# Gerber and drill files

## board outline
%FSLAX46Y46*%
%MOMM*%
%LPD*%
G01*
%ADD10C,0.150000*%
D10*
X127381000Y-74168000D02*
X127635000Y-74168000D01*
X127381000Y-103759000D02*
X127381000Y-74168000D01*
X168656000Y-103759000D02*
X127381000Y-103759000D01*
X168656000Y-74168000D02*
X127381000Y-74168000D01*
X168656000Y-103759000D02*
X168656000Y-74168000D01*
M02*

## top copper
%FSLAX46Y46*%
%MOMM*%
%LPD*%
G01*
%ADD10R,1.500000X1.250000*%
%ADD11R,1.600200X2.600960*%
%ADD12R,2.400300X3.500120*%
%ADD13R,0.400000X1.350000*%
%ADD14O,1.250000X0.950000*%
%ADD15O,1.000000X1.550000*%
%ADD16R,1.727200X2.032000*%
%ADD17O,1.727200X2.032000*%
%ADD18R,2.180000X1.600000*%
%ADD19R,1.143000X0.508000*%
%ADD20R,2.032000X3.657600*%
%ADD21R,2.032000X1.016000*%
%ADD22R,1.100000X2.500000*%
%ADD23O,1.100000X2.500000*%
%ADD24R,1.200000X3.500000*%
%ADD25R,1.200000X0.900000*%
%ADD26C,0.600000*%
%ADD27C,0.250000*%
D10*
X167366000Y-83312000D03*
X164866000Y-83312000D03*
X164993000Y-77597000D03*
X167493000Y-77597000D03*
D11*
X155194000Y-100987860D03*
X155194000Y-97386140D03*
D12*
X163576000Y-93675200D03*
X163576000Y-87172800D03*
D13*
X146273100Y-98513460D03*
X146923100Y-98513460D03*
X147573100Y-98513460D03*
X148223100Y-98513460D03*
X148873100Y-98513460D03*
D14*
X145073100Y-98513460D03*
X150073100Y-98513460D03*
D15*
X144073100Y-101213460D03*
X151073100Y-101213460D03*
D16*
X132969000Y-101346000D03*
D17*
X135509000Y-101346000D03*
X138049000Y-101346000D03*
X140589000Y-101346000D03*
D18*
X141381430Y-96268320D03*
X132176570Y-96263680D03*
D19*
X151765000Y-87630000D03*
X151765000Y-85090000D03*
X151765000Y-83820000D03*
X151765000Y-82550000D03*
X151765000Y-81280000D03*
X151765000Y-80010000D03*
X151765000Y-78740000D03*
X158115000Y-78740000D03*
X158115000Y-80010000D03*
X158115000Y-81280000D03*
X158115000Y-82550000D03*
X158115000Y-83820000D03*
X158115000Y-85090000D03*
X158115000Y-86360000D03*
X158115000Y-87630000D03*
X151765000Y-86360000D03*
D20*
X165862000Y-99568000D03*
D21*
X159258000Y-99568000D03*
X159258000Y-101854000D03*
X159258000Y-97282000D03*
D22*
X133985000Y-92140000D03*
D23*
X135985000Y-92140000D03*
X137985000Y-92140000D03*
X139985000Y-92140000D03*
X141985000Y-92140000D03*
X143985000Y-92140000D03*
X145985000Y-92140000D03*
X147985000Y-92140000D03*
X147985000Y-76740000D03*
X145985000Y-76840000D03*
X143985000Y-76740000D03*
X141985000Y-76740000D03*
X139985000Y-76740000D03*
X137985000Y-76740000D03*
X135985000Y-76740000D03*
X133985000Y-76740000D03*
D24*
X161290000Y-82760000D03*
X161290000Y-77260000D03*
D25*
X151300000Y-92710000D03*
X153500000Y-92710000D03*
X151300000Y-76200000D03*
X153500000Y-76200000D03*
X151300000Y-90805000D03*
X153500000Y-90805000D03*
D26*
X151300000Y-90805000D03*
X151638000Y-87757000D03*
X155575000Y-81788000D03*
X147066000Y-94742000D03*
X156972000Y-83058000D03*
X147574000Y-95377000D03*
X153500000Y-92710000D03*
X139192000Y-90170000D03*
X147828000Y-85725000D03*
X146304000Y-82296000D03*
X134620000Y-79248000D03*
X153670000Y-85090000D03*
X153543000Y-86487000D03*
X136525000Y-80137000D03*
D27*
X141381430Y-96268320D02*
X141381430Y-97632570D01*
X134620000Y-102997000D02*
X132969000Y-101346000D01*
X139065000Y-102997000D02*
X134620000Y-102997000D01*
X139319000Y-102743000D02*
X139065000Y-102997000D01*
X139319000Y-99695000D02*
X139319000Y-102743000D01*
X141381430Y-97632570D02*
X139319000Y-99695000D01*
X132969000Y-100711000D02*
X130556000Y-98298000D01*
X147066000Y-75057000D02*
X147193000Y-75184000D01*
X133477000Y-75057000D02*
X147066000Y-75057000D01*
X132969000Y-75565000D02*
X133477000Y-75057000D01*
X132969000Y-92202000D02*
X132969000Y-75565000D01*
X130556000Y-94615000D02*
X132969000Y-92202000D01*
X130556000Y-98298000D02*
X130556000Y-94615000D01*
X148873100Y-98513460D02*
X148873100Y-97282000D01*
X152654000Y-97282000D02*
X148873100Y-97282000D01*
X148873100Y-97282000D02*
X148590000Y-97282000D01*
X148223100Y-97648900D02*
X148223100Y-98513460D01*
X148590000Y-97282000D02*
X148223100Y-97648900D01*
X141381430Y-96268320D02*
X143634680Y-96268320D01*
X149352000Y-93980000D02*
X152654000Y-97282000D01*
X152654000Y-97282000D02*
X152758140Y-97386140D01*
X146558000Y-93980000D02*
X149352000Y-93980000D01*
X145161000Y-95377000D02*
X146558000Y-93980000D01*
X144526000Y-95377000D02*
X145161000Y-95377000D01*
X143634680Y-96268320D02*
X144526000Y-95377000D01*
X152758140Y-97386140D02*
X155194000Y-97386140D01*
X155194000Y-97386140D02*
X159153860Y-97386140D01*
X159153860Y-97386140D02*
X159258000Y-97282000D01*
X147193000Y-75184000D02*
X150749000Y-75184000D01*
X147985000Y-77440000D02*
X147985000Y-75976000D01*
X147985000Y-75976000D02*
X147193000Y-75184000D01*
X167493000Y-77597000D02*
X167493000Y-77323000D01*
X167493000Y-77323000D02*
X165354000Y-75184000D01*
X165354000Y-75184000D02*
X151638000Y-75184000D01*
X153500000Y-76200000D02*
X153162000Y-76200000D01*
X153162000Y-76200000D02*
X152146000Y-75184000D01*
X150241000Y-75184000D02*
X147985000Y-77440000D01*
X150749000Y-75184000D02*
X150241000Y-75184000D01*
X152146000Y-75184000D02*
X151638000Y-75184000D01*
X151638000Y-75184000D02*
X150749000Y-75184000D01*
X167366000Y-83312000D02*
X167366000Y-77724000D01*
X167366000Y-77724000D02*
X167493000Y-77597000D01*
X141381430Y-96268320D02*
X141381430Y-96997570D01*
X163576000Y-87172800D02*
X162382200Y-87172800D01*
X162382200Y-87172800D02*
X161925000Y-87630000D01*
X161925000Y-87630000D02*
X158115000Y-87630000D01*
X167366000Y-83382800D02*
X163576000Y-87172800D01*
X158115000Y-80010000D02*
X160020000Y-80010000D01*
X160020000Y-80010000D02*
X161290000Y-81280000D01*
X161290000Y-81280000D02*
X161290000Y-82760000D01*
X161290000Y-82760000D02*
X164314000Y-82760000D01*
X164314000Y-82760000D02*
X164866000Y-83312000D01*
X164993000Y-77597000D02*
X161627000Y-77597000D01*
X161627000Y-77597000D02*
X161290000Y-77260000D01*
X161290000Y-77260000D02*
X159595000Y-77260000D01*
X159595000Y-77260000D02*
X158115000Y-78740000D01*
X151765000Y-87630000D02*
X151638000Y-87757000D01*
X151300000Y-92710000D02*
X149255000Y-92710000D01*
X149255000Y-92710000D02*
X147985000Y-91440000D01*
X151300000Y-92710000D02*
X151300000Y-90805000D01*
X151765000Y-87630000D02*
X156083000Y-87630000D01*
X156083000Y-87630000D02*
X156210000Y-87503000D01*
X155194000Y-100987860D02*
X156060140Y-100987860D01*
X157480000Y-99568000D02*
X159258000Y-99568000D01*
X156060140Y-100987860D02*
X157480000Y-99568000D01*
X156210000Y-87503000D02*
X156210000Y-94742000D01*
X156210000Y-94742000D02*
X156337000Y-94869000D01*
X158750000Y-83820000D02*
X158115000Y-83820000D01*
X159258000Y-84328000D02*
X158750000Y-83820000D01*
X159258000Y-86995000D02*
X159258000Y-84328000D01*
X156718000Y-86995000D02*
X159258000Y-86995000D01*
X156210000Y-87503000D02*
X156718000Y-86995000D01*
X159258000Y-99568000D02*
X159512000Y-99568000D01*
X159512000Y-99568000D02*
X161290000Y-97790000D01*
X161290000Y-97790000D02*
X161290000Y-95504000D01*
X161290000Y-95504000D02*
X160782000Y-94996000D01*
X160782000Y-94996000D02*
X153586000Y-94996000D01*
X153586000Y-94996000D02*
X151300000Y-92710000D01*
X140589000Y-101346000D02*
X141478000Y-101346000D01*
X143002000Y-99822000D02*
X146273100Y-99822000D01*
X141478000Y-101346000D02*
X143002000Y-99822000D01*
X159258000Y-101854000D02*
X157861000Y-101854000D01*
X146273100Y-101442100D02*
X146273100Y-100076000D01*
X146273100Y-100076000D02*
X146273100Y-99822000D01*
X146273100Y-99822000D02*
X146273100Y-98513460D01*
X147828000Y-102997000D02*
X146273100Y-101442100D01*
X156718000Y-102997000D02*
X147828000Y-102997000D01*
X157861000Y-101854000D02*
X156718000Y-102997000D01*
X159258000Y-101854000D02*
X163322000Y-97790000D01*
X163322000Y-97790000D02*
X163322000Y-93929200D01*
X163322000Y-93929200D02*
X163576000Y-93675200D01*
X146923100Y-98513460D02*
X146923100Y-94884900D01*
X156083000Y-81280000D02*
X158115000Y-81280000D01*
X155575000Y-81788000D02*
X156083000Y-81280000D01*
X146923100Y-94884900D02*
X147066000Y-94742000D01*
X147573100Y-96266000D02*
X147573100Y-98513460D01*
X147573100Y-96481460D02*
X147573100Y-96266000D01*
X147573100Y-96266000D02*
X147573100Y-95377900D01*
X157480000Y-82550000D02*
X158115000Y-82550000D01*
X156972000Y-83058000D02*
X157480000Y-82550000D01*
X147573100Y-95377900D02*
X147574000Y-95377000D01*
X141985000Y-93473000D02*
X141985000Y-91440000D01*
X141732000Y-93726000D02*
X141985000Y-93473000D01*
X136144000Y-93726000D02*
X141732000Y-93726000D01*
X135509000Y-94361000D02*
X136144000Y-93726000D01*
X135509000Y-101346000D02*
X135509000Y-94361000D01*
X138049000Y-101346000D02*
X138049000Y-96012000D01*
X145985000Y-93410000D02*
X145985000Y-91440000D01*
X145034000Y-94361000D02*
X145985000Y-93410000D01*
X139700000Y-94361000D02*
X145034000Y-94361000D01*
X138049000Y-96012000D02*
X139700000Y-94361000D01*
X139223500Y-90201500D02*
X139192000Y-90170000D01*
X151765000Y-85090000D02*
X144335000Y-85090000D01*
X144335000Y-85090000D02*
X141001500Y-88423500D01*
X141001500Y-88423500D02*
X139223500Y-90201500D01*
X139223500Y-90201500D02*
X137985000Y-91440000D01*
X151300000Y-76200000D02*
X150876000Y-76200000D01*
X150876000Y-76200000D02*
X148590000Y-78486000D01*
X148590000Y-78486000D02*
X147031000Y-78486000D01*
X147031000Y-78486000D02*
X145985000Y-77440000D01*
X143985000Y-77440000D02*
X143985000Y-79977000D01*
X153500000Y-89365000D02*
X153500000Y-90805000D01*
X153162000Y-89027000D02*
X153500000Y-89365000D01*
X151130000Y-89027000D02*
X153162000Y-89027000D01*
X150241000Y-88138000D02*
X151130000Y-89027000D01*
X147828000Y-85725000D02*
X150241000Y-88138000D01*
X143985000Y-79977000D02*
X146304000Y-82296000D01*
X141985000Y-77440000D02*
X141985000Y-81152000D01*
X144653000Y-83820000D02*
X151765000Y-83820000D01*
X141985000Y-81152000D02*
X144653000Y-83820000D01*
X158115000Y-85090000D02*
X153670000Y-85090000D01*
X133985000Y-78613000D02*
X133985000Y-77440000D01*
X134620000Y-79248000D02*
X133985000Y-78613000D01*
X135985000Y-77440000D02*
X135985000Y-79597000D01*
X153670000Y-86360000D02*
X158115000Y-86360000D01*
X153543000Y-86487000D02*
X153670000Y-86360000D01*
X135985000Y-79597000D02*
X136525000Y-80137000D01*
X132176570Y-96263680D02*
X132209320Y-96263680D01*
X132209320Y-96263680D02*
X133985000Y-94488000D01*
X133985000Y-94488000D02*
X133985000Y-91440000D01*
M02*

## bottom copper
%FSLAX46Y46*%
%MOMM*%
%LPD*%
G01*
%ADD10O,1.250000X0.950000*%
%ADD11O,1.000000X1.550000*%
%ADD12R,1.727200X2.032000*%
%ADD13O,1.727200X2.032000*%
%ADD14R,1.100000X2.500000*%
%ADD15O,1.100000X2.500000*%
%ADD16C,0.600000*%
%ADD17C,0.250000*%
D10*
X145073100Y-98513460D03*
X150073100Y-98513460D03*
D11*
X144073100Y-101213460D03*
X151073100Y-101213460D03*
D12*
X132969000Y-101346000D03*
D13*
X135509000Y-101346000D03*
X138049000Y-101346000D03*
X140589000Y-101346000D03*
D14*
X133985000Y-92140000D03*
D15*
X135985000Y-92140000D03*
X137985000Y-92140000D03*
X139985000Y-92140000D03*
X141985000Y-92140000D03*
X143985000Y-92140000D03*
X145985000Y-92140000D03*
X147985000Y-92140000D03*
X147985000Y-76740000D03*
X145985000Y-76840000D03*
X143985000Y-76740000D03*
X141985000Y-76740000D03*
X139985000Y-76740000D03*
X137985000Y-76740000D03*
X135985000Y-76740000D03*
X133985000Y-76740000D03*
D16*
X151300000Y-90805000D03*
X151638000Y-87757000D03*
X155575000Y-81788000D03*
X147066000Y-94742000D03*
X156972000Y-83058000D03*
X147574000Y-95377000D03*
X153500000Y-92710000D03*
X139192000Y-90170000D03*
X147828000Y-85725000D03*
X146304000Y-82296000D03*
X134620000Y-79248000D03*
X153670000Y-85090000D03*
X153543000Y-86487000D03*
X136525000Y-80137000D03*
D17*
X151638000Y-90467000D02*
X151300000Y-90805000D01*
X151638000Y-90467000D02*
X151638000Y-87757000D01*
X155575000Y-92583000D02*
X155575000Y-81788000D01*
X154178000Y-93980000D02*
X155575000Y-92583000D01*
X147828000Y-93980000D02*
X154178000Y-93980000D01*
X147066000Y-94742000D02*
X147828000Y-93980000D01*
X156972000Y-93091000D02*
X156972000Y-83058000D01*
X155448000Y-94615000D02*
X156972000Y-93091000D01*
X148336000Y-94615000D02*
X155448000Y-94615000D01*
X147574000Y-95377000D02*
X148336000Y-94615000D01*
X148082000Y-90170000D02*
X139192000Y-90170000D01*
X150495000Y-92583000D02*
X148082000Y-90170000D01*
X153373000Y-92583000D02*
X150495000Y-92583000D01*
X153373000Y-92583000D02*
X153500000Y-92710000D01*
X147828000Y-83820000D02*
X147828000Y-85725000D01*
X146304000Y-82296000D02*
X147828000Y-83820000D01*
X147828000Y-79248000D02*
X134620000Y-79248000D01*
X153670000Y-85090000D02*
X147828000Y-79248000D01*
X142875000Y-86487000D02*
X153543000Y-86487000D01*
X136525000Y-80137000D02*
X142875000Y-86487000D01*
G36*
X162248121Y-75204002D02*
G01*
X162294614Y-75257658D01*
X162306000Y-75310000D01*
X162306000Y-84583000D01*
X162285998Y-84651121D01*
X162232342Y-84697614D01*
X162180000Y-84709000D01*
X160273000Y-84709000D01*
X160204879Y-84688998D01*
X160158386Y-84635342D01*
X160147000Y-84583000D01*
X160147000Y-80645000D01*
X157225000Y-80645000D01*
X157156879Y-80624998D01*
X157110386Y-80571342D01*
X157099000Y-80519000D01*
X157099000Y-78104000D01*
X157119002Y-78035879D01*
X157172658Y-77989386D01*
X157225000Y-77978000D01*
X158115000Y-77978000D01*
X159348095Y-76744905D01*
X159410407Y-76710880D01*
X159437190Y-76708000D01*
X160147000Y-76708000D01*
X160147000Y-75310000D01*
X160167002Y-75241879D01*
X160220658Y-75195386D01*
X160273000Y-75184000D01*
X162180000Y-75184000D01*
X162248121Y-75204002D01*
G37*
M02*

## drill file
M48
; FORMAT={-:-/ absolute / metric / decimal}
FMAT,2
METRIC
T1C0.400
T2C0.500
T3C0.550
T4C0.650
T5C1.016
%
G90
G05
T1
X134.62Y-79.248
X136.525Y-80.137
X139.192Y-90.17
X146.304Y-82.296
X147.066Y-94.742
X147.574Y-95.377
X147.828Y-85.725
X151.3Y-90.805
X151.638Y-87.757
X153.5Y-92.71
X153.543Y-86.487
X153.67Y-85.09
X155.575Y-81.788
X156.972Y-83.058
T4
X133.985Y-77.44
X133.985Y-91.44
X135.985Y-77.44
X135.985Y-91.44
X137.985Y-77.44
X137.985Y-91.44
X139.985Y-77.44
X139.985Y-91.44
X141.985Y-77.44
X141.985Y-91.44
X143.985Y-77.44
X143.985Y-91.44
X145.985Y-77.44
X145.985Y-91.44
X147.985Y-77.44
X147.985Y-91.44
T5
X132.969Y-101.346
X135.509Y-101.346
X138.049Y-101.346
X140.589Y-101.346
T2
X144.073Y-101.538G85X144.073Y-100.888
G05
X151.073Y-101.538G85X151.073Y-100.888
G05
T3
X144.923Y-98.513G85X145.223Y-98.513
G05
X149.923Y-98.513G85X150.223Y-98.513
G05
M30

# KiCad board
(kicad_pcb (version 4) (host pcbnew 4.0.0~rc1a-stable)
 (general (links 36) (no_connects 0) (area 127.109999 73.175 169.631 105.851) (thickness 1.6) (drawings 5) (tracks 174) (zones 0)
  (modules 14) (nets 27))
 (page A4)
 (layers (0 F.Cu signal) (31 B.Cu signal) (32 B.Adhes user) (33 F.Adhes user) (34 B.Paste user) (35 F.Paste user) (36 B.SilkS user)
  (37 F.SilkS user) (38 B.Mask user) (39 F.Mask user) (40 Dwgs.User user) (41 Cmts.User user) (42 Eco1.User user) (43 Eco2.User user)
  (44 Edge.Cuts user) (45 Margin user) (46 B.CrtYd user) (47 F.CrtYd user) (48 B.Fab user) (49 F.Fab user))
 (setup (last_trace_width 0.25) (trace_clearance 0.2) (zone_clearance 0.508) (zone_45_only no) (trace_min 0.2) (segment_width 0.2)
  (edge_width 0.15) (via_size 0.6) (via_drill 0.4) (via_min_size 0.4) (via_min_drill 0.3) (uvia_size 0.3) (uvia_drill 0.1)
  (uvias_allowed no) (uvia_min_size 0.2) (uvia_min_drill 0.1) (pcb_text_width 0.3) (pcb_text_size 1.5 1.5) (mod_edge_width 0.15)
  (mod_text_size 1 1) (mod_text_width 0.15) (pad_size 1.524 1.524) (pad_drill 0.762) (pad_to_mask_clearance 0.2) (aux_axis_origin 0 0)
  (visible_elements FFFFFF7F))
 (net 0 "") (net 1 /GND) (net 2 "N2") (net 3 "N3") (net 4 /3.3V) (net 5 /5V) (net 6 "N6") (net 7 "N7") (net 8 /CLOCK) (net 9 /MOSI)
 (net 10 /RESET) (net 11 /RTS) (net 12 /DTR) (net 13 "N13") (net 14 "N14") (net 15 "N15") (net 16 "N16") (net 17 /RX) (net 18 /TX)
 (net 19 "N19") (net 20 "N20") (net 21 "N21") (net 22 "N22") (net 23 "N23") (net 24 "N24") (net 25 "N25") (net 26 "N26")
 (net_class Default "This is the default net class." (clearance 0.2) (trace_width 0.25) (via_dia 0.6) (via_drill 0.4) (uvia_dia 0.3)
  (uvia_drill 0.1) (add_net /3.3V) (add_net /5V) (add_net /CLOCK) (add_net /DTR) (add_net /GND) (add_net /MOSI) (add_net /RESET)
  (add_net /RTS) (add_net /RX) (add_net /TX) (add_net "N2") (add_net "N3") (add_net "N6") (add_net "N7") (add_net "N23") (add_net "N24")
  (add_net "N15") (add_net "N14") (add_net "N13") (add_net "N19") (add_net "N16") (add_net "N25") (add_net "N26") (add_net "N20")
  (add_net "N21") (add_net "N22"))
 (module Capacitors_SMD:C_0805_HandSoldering (layer F.Cu) (at 166.116 83.312 180)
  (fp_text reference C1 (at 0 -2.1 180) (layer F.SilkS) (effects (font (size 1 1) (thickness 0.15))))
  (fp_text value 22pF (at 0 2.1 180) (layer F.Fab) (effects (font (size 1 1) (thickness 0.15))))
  (pad 1 smd rect (at -1.25 0 180) (size 1.5 1.25) (layers F.Cu F.Paste F.Mask) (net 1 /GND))
  (pad 2 smd rect (at 1.25 0 180) (size 1.5 1.25) (layers F.Cu F.Paste F.Mask) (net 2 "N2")))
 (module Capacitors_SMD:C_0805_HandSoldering (layer F.Cu) (at 166.243 77.597)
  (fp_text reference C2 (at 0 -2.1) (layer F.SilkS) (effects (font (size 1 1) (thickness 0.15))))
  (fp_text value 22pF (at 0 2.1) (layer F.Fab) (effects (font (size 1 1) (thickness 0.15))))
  (pad 1 smd rect (at -1.25 0) (size 1.5 1.25) (layers F.Cu F.Paste F.Mask) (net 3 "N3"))
  (pad 2 smd rect (at 1.25 0) (size 1.5 1.25) (layers F.Cu F.Paste F.Mask) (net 1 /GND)))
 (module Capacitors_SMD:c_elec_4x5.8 (layer F.Cu) (at 155.194 99.187 270)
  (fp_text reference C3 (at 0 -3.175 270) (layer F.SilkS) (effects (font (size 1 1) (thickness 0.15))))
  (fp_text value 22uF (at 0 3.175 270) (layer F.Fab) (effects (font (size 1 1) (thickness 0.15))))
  (pad 1 smd rect (at 1.80086 0 270) (size 2.60096 1.6002) (layers F.Cu F.Paste F.Mask) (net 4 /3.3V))
  (pad 2 smd rect (at -1.80086 0 270) (size 2.60096 1.6002) (layers F.Cu F.Paste F.Mask) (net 1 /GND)))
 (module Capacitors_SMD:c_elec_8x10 (layer F.Cu) (at 163.576 90.424 270)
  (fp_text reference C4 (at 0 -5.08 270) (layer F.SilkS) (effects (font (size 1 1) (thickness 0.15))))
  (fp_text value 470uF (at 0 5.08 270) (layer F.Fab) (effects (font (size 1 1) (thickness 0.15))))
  (pad 1 smd rect (at 3.2512 0 270) (size 3.50012 2.4003) (layers F.Cu F.Paste F.Mask) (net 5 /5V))
  (pad 2 smd rect (at -3.2512 0 270) (size 3.50012 2.4003) (layers F.Cu F.Paste F.Mask) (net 1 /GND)))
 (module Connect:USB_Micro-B (layer F.Cu) (at 147.574 100.076)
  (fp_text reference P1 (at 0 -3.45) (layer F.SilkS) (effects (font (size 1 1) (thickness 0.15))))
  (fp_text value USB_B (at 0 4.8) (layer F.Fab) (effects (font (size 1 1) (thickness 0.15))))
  (pad 1 smd rect (at -1.3009 -1.56254 90) (size 1.35 0.4) (layers F.Cu F.Paste F.Mask) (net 5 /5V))
  (pad 2 smd rect (at -0.6509 -1.56254 90) (size 1.35 0.4) (layers F.Cu F.Paste F.Mask) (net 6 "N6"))
  (pad 3 smd rect (at -0.0009 -1.56254 90) (size 1.35 0.4) (layers F.Cu F.Paste F.Mask) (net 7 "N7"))
  (pad 4 smd rect (at 0.6491 -1.56254 90) (size 1.35 0.4) (layers F.Cu F.Paste F.Mask) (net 1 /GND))
  (pad 5 smd rect (at 1.2991 -1.56254 90) (size 1.35 0.4) (layers F.Cu F.Paste F.Mask) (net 1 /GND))
  (pad 6 thru_hole oval (at -2.5009 -1.56254 90) (size 0.95 1.25) (drill oval 0.55 0.85) (layers *.Cu *.Mask F.SilkS))
  (pad 6 thru_hole oval (at 2.4991 -1.56254 90) (size 0.95 1.25) (drill oval 0.55 0.85) (layers *.Cu *.Mask F.SilkS))
  (pad 6 thru_hole oval (at -3.5009 1.13746 90) (size 1.55 1) (drill oval 1.15 0.5) (layers *.Cu *.Mask F.SilkS))
  (pad 6 thru_hole oval (at 3.4991 1.13746 90) (size 1.55 1) (drill oval 1.15 0.5) (layers *.Cu *.Mask F.SilkS)))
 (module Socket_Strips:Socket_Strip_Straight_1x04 (layer F.Cu) (at 132.969 101.346)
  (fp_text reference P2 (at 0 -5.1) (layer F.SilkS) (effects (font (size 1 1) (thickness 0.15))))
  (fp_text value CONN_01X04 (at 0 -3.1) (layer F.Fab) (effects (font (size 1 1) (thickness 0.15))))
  (pad 1 thru_hole rect (at 0 0) (size 1.7272 2.032) (drill 1.016) (layers *.Cu *.Mask F.SilkS) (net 1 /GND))
  (pad 2 thru_hole oval (at 2.54 0) (size 1.7272 2.032) (drill 1.016) (layers *.Cu *.Mask F.SilkS) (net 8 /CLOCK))
  (pad 3 thru_hole oval (at 5.08 0) (size 1.7272 2.032) (drill 1.016) (layers *.Cu *.Mask F.SilkS) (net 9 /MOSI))
  (pad 4 thru_hole oval (at 7.62 0) (size 1.7272 2.032) (drill 1.016) (layers *.Cu *.Mask F.SilkS) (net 5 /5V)))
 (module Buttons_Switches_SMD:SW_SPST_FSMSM (layer F.Cu) (at 136.779 96.266 180)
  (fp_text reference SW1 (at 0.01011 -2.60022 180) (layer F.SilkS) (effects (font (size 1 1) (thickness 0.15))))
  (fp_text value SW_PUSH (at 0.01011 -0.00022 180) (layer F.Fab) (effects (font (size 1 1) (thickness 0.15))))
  (pad 1 smd rect (at -4.60243 -0.00232 180) (size 2.18 1.6) (layers F.Cu F.Paste F.Mask) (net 1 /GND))
  (pad 2 smd rect (at 4.60243 0.00232 180) (size 2.18 1.6) (layers F.Cu F.Paste F.Mask) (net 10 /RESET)))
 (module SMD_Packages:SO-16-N (layer F.Cu) (at 154.94 83.185 90)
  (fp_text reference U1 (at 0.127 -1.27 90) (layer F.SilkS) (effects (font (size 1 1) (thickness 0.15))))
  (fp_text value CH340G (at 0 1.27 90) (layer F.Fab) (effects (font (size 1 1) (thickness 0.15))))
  (pad 16 smd rect (at -4.445 -3.175 90) (size 0.508 1.143) (layers F.Cu F.Paste F.Mask) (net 4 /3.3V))
  (pad 14 smd rect (at -1.905 -3.175 90) (size 0.508 1.143) (layers F.Cu F.Paste F.Mask) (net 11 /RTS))
  (pad 13 smd rect (at -0.635 -3.175 90) (size 0.508 1.143) (layers F.Cu F.Paste F.Mask) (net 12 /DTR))
  (pad 12 smd rect (at 0.635 -3.175 90) (size 0.508 1.143) (layers F.Cu F.Paste F.Mask) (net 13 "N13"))
  (pad 11 smd rect (at 1.905 -3.175 90) (size 0.508 1.143) (layers F.Cu F.Paste F.Mask) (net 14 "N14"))
  (pad 10 smd rect (at 3.175 -3.175 90) (size 0.508 1.143) (layers F.Cu F.Paste F.Mask) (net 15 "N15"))
  (pad 9 smd rect (at 4.445 -3.175 90) (size 0.508 1.143) (layers F.Cu F.Paste F.Mask) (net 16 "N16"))
  (pad 8 smd rect (at 4.445 3.175 90) (size 0.508 1.143) (layers F.Cu F.Paste F.Mask) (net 3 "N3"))
  (pad 7 smd rect (at 3.175 3.175 90) (size 0.508 1.143) (layers F.Cu F.Paste F.Mask) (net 2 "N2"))
  (pad 6 smd rect (at 1.905 3.175 90) (size 0.508 1.143) (layers F.Cu F.Paste F.Mask) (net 6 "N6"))
  (pad 5 smd rect (at 0.635 3.175 90) (size 0.508 1.143) (layers F.Cu F.Paste F.Mask) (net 7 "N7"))
  (pad 4 smd rect (at -0.635 3.175 90) (size 0.508 1.143) (layers F.Cu F.Paste F.Mask) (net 4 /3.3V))
  (pad 3 smd rect (at -1.905 3.175 90) (size 0.508 1.143) (layers F.Cu F.Paste F.Mask) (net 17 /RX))
  (pad 2 smd rect (at -3.175 3.175 90) (size 0.508 1.143) (layers F.Cu F.Paste F.Mask) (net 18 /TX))
  (pad 1 smd rect (at -4.445 3.175 90) (size 0.508 1.143) (layers F.Cu F.Paste F.Mask) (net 1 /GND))
  (pad 15 smd rect (at -3.175 -3.175 90) (size 0.508 1.143) (layers F.Cu F.Paste F.Mask) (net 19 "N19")))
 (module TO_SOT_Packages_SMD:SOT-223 (layer F.Cu) (at 162.56 99.568 270)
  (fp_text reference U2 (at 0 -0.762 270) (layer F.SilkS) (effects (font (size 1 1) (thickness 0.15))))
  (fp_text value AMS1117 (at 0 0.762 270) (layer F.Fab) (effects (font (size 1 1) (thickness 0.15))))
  (pad 4 smd rect (at 0 -3.302 270) (size 3.6576 2.032) (layers F.Cu F.Paste F.Mask))
  (pad 2 smd rect (at 0 3.302 270) (size 1.016 2.032) (layers F.Cu F.Paste F.Mask) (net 4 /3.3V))
  (pad 3 smd rect (at 2.286 3.302 270) (size 1.016 2.032) (layers F.Cu F.Paste F.Mask) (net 5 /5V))
  (pad 1 smd rect (at -2.286 3.302 270) (size 1.016 2.032) (layers F.Cu F.Paste F.Mask) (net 1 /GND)))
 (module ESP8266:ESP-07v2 (layer F.Cu) (at 133.985 91.44 90)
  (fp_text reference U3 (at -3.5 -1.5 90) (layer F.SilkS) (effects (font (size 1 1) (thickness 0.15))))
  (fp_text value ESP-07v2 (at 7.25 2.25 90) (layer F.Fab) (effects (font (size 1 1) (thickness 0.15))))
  (pad 1 thru_hole rect (at 0 0 90) (size 2.5 1.1) (drill 0.65 (offset -0.7 0)) (layers *.Cu *.Mask F.SilkS) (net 10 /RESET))
  (pad 2 thru_hole oval (at 0 2 90) (size 2.5 1.1) (drill 0.65 (offset -0.7 0)) (layers *.Cu *.Mask F.SilkS) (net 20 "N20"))
  (pad 3 thru_hole oval (at 0 4 90) (size 2.5 1.1) (drill 0.65 (offset -0.7 0)) (layers *.Cu *.Mask F.SilkS) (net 11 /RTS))
  (pad 4 thru_hole oval (at 0 6 90) (size 2.5 1.1) (drill 0.65 (offset -0.7 0)) (layers *.Cu *.Mask F.SilkS) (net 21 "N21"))
  (pad 5 thru_hole oval (at 0 8 90) (size 2.5 1.1) (drill 0.65 (offset -0.7 0)) (layers *.Cu *.Mask F.SilkS) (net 8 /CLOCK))
  (pad 6 thru_hole oval (at 0 10 90) (size 2.5 1.1) (drill 0.65 (offset -0.7 0)) (layers *.Cu *.Mask F.SilkS) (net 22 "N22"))
  (pad 7 thru_hole oval (at 0 12 90) (size 2.5 1.1) (drill 0.65 (offset -0.7 0)) (layers *.Cu *.Mask F.SilkS) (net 9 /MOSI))
  (pad 8 thru_hole oval (at 0 14 90) (size 2.5 1.1) (drill 0.65 (offset -0.7 0)) (layers *.Cu *.Mask F.SilkS) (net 4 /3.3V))
  (pad 9 thru_hole oval (at 14 14 90) (size 2.5 1.1) (drill 0.65 (offset 0.7 0)) (layers *.Cu *.Mask F.SilkS) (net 1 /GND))
  (pad 10 thru_hole oval (at 14 12 90) (size 2.5 1.1) (drill 0.65 (offset 0.6 0)) (layers *.Cu *.Mask F.SilkS) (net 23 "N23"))
  (pad 11 thru_hole oval (at 14 10 90) (size 2.5 1.1) (drill 0.65 (offset 0.7 0)) (layers *.Cu *.Mask F.SilkS) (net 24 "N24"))
  (pad 12 thru_hole oval (at 14 8 90) (size 2.5 1.1) (drill 0.65 (offset 0.7 0)) (layers *.Cu *.Mask F.SilkS) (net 12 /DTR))
  (pad 13 thru_hole oval (at 14 6 90) (size 2.5 1.1) (drill 0.65 (offset 0.7 0)) (layers *.Cu *.Mask F.SilkS) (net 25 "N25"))
  (pad 14 thru_hole oval (at 14 4 90) (size 2.5 1.1) (drill 0.65 (offset 0.7 0)) (layers *.Cu *.Mask F.SilkS) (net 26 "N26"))
  (pad 15 thru_hole oval (at 14 2 90) (size 2.5 1.1) (drill 0.65 (offset 0.7 0)) (layers *.Cu *.Mask F.SilkS) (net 18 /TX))
  (pad 16 thru_hole oval (at 14 0 90) (size 2.5 1.1) (drill 0.65 (offset 0.7 0)) (layers *.Cu *.Mask F.SilkS) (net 17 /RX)))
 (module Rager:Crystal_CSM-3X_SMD (layer F.Cu) (at 161.29 80.01 90)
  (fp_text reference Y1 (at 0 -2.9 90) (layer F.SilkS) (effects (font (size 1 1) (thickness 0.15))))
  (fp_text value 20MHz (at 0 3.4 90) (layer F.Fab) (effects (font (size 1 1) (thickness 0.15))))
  (pad 1 smd rect (at -2.75 0 90) (size 3.5 1.2) (layers F.Cu F.Paste F.Mask) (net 2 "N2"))
  (pad 2 smd rect (at 2.75 0 90) (size 3.5 1.2) (layers F.Cu F.Paste F.Mask) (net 3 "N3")))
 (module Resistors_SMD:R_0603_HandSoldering (layer F.Cu) (at 152.4 92.71)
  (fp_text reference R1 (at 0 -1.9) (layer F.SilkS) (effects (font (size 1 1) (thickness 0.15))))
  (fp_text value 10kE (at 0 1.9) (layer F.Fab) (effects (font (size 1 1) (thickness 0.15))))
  (pad 1 smd rect (at -1.1 0) (size 1.2 0.9) (layers F.Cu F.Paste F.Mask) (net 4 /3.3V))
  (pad 2 smd rect (at 1.1 0) (size 1.2 0.9) (layers F.Cu F.Paste F.Mask) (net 11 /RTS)))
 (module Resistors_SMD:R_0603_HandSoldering (layer F.Cu) (at 152.4 76.2)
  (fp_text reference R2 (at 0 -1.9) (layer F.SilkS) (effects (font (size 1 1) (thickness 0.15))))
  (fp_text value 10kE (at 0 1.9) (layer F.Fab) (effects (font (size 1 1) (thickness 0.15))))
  (pad 1 smd rect (at -1.1 0) (size 1.2 0.9) (layers F.Cu F.Paste F.Mask) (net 23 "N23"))
  (pad 2 smd rect (at 1.1 0) (size 1.2 0.9) (layers F.Cu F.Paste F.Mask) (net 1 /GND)))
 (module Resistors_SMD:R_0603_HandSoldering (layer F.Cu) (at 152.4 90.805)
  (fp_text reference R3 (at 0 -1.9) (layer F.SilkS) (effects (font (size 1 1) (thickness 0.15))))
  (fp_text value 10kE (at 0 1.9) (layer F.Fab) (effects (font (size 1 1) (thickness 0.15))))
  (pad 1 smd rect (at -1.1 0) (size 1.2 0.9) (layers F.Cu F.Paste F.Mask) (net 4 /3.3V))
  (pad 2 smd rect (at 1.1 0) (size 1.2 0.9) (layers F.Cu F.Paste F.Mask) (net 24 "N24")))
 (gr_line (start 127.381 74.168) (end 127.635 74.168) (angle 90) (layer Edge.Cuts) (width 0.15))
 (gr_line (start 127.381 103.759) (end 127.381 74.168) (angle 90) (layer Edge.Cuts) (width 0.15))
 (gr_line (start 168.656 103.759) (end 127.381 103.759) (angle 90) (layer Edge.Cuts) (width 0.15))
 (gr_line (start 168.656 74.168) (end 127.381 74.168) (angle 90) (layer Edge.Cuts) (width 0.15))
 (gr_line (start 168.656 103.759) (end 168.656 74.168) (angle 90) (layer Edge.Cuts) (width 0.15))
 (segment (start 141.38143 96.26832) (end 141.38143 97.63257) (width 0.25) (layer F.Cu) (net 1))
 (segment (start 134.62 102.997) (end 132.969 101.346) (width 0.25) (layer F.Cu) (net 1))
 (segment (start 139.065 102.997) (end 134.62 102.997) (width 0.25) (layer F.Cu) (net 1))
 (segment (start 139.319 102.743) (end 139.065 102.997) (width 0.25) (layer F.Cu) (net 1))
 (segment (start 139.319 99.695) (end 139.319 102.743) (width 0.25) (layer F.Cu) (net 1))
 (segment (start 141.38143 97.63257) (end 139.319 99.695) (width 0.25) (layer F.Cu) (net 1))
 (segment (start 132.969 100.711) (end 130.556 98.298) (width 0.25) (layer F.Cu) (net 1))
 (segment (start 147.066 75.057) (end 147.193 75.184) (width 0.25) (layer F.Cu) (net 1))
 (segment (start 133.477 75.057) (end 147.066 75.057) (width 0.25) (layer F.Cu) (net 1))
 (segment (start 132.969 75.565) (end 133.477 75.057) (width 0.25) (layer F.Cu) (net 1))
 (segment (start 132.969 92.202) (end 132.969 75.565) (width 0.25) (layer F.Cu) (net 1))
 (segment (start 130.556 94.615) (end 132.969 92.202) (width 0.25) (layer F.Cu) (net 1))
 (segment (start 130.556 98.298) (end 130.556 94.615) (width 0.25) (layer F.Cu) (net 1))
 (segment (start 148.8731 98.51346) (end 148.8731 97.282) (width 0.25) (layer F.Cu) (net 1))
 (segment (start 152.654 97.282) (end 148.8731 97.282) (width 0.25) (layer F.Cu) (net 1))
 (segment (start 148.8731 97.282) (end 148.59 97.282) (width 0.25) (layer F.Cu) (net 1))
 (segment (start 148.2231 97.6489) (end 148.2231 98.51346) (width 0.25) (layer F.Cu) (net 1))
 (segment (start 148.59 97.282) (end 148.2231 97.6489) (width 0.25) (layer F.Cu) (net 1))
 (segment (start 141.38143 96.26832) (end 143.63468 96.26832) (width 0.25) (layer F.Cu) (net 1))
 (segment (start 149.352 93.98) (end 152.654 97.282) (width 0.25) (layer F.Cu) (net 1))
 (segment (start 152.654 97.282) (end 152.75814 97.38614) (width 0.25) (layer F.Cu) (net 1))
 (segment (start 146.558 93.98) (end 149.352 93.98) (width 0.25) (layer F.Cu) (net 1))
 (segment (start 145.161 95.377) (end 146.558 93.98) (width 0.25) (layer F.Cu) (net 1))
 (segment (start 144.526 95.377) (end 145.161 95.377) (width 0.25) (layer F.Cu) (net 1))
 (segment (start 143.63468 96.26832) (end 144.526 95.377) (width 0.25) (layer F.Cu) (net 1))
 (segment (start 152.75814 97.38614) (end 155.194 97.38614) (width 0.25) (layer F.Cu) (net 1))
 (segment (start 155.194 97.38614) (end 159.15386 97.38614) (width 0.25) (layer F.Cu) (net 1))
 (segment (start 159.15386 97.38614) (end 159.258 97.282) (width 0.25) (layer F.Cu) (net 1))
 (segment (start 147.193 75.184) (end 150.749 75.184) (width 0.25) (layer F.Cu) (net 1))
 (segment (start 147.985 77.44) (end 147.985 75.976) (width 0.25) (layer F.Cu) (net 1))
 (segment (start 147.985 75.976) (end 147.193 75.184) (width 0.25) (layer F.Cu) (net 1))
 (segment (start 167.493 77.597) (end 167.493 77.323) (width 0.25) (layer F.Cu) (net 1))
 (segment (start 167.493 77.323) (end 165.354 75.184) (width 0.25) (layer F.Cu) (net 1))
 (segment (start 165.354 75.184) (end 151.638 75.184) (width 0.25) (layer F.Cu) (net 1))
 (segment (start 153.5 76.2) (end 153.162 76.2) (width 0.25) (layer F.Cu) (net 1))
 (segment (start 153.162 76.2) (end 152.146 75.184) (width 0.25) (layer F.Cu) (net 1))
 (segment (start 150.241 75.184) (end 147.985 77.44) (width 0.25) (layer F.Cu) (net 1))
 (segment (start 150.749 75.184) (end 150.241 75.184) (width 0.25) (layer F.Cu) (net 1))
 (segment (start 152.146 75.184) (end 151.638 75.184) (width 0.25) (layer F.Cu) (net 1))
 (segment (start 151.638 75.184) (end 150.749 75.184) (width 0.25) (layer F.Cu) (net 1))
 (segment (start 167.366 83.312) (end 167.366 77.724) (width 0.25) (layer F.Cu) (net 1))
 (segment (start 167.366 77.724) (end 167.493 77.597) (width 0.25) (layer F.Cu) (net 1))
 (segment (start 141.38143 96.26832) (end 141.38143 96.99757) (width 0.25) (layer F.Cu) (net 1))
 (segment (start 163.576 87.1728) (end 162.3822 87.1728) (width 0.25) (layer F.Cu) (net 1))
 (segment (start 162.3822 87.1728) (end 161.925 87.63) (width 0.25) (layer F.Cu) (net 1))
 (segment (start 161.925 87.63) (end 158.115 87.63) (width 0.25) (layer F.Cu) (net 1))
 (segment (start 167.366 83.3828) (end 163.576 87.1728) (width 0.25) (layer F.Cu) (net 1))
 (segment (start 158.115 80.01) (end 160.02 80.01) (width 0.25) (layer F.Cu) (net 2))
 (segment (start 160.02 80.01) (end 161.29 81.28) (width 0.25) (layer F.Cu) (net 2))
 (segment (start 161.29 81.28) (end 161.29 82.76) (width 0.25) (layer F.Cu) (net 2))
 (segment (start 161.29 82.76) (end 164.314 82.76) (width 0.25) (layer F.Cu) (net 2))
 (segment (start 164.314 82.76) (end 164.866 83.312) (width 0.25) (layer F.Cu) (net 2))
 (segment (start 164.993 77.597) (end 161.627 77.597) (width 0.25) (layer F.Cu) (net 3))
 (segment (start 161.627 77.597) (end 161.29 77.26) (width 0.25) (layer F.Cu) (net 3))
 (segment (start 161.29 77.26) (end 159.595 77.26) (width 0.25) (layer F.Cu) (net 3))
 (segment (start 159.595 77.26) (end 158.115 78.74) (width 0.25) (layer F.Cu) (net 3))
 (via (at 151.3 90.805) (size 0.6) (drill 0.4) (layers F.Cu B.Cu) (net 4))
 (segment (start 151.638 90.467) (end 151.3 90.805) (width 0.25) (layer B.Cu) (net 4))
 (segment (start 151.638 90.467) (end 151.638 87.757) (width 0.25) (layer B.Cu) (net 4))
 (via (at 151.638 87.757) (size 0.6) (drill 0.4) (layers F.Cu B.Cu) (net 4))
 (segment (start 151.765 87.63) (end 151.638 87.757) (width 0.25) (layer F.Cu) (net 4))
 (segment (start 151.3 92.71) (end 149.255 92.71) (width 0.25) (layer F.Cu) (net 4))
 (segment (start 149.255 92.71) (end 147.985 91.44) (width 0.25) (layer F.Cu) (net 4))
 (segment (start 151.3 92.71) (end 151.3 90.805) (width 0.25) (layer F.Cu) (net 4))
 (segment (start 151.765 87.63) (end 156.083 87.63) (width 0.25) (layer F.Cu) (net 4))
 (segment (start 156.083 87.63) (end 156.21 87.503) (width 0.25) (layer F.Cu) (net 4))
 (segment (start 155.194 100.98786) (end 156.06014 100.98786) (width 0.25) (layer F.Cu) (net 4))
 (segment (start 157.48 99.568) (end 159.258 99.568) (width 0.25) (layer F.Cu) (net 4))
 (segment (start 156.06014 100.98786) (end 157.48 99.568) (width 0.25) (layer F.Cu) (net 4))
 (segment (start 156.21 87.503) (end 156.21 94.742) (width 0.25) (layer F.Cu) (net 4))
 (segment (start 156.21 94.742) (end 156.337 94.869) (width 0.25) (layer F.Cu) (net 4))
 (segment (start 158.75 83.82) (end 158.115 83.82) (width 0.25) (layer F.Cu) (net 4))
 (segment (start 159.258 84.328) (end 158.75 83.82) (width 0.25) (layer F.Cu) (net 4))
 (segment (start 159.258 86.995) (end 159.258 84.328) (width 0.25) (layer F.Cu) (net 4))
 (segment (start 156.718 86.995) (end 159.258 86.995) (width 0.25) (layer F.Cu) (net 4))
 (segment (start 156.21 87.503) (end 156.718 86.995) (width 0.25) (layer F.Cu) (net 4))
 (segment (start 159.258 99.568) (end 159.512 99.568) (width 0.25) (layer F.Cu) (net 4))
 (segment (start 159.512 99.568) (end 161.29 97.79) (width 0.25) (layer F.Cu) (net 4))
 (segment (start 161.29 97.79) (end 161.29 95.504) (width 0.25) (layer F.Cu) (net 4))
 (segment (start 161.29 95.504) (end 160.782 94.996) (width 0.25) (layer F.Cu) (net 4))
 (segment (start 160.782 94.996) (end 153.586 94.996) (width 0.25) (layer F.Cu) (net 4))
 (segment (start 153.586 94.996) (end 151.3 92.71) (width 0.25) (layer F.Cu) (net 4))
 (segment (start 140.589 101.346) (end 141.478 101.346) (width 0.25) (layer F.Cu) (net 5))
 (segment (start 143.002 99.822) (end 146.2731 99.822) (width 0.25) (layer F.Cu) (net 5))
 (segment (start 141.478 101.346) (end 143.002 99.822) (width 0.25) (layer F.Cu) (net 5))
 (segment (start 159.258 101.854) (end 157.861 101.854) (width 0.25) (layer F.Cu) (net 5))
 (segment (start 146.2731 101.4421) (end 146.2731 100.076) (width 0.25) (layer F.Cu) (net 5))
 (segment (start 146.2731 100.076) (end 146.2731 99.822) (width 0.25) (layer F.Cu) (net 5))
 (segment (start 146.2731 99.822) (end 146.2731 98.51346) (width 0.25) (layer F.Cu) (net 5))
 (segment (start 147.828 102.997) (end 146.2731 101.4421) (width 0.25) (layer F.Cu) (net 5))
 (segment (start 156.718 102.997) (end 147.828 102.997) (width 0.25) (layer F.Cu) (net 5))
 (segment (start 157.861 101.854) (end 156.718 102.997) (width 0.25) (layer F.Cu) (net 5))
 (segment (start 159.258 101.854) (end 163.322 97.79) (width 0.25) (layer F.Cu) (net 5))
 (segment (start 163.322 97.79) (end 163.322 93.9292) (width 0.25) (layer F.Cu) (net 5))
 (segment (start 163.322 93.9292) (end 163.576 93.6752) (width 0.25) (layer F.Cu) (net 5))
 (segment (start 146.9231 98.51346) (end 146.9231 94.8849) (width 0.25) (layer F.Cu) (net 6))
 (segment (start 156.083 81.28) (end 158.115 81.28) (width 0.25) (layer F.Cu) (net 6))
 (segment (start 155.575 81.788) (end 156.083 81.28) (width 0.25) (layer F.Cu) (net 6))
 (via (at 155.575 81.788) (size 0.6) (drill 0.4) (layers F.Cu B.Cu) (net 6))
 (segment (start 155.575 92.583) (end 155.575 81.788) (width 0.25) (layer B.Cu) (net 6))
 (segment (start 154.178 93.98) (end 155.575 92.583) (width 0.25) (layer B.Cu) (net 6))
 (segment (start 147.828 93.98) (end 154.178 93.98) (width 0.25) (layer B.Cu) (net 6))
 (segment (start 147.066 94.742) (end 147.828 93.98) (width 0.25) (layer B.Cu) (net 6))
 (via (at 147.066 94.742) (size 0.6) (drill 0.4) (layers F.Cu B.Cu) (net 6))
 (segment (start 146.9231 94.8849) (end 147.066 94.742) (width 0.25) (layer F.Cu) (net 6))
 (segment (start 147.5731 96.266) (end 147.5731 98.51346) (width 0.25) (layer F.Cu) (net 7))
 (segment (start 147.5731 96.48146) (end 147.5731 96.266) (width 0.25) (layer F.Cu) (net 7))
 (segment (start 147.5731 96.266) (end 147.5731 95.3779) (width 0.25) (layer F.Cu) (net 7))
 (segment (start 157.48 82.55) (end 158.115 82.55) (width 0.25) (layer F.Cu) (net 7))
 (segment (start 156.972 83.058) (end 157.48 82.55) (width 0.25) (layer F.Cu) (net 7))
 (via (at 156.972 83.058) (size 0.6) (drill 0.4) (layers F.Cu B.Cu) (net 7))
 (segment (start 156.972 93.091) (end 156.972 83.058) (width 0.25) (layer B.Cu) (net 7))
 (segment (start 155.448 94.615) (end 156.972 93.091) (width 0.25) (layer B.Cu) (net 7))
 (segment (start 148.336 94.615) (end 155.448 94.615) (width 0.25) (layer B.Cu) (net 7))
 (segment (start 147.574 95.377) (end 148.336 94.615) (width 0.25) (layer B.Cu) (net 7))
 (via (at 147.574 95.377) (size 0.6) (drill 0.4) (layers F.Cu B.Cu) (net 7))
 (segment (start 147.5731 95.3779) (end 147.574 95.377) (width 0.25) (layer F.Cu) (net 7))
 (segment (start 141.985 93.473) (end 141.985 91.44) (width 0.25) (layer F.Cu) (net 8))
 (segment (start 141.732 93.726) (end 141.985 93.473) (width 0.25) (layer F.Cu) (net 8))
 (segment (start 136.144 93.726) (end 141.732 93.726) (width 0.25) (layer F.Cu) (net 8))
 (segment (start 135.509 94.361) (end 136.144 93.726) (width 0.25) (layer F.Cu) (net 8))
 (segment (start 135.509 101.346) (end 135.509 94.361) (width 0.25) (layer F.Cu) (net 8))
 (segment (start 138.049 101.346) (end 138.049 96.012) (width 0.25) (layer F.Cu) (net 9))
 (segment (start 145.985 93.41) (end 145.985 91.44) (width 0.25) (layer F.Cu) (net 9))
 (segment (start 145.034 94.361) (end 145.985 93.41) (width 0.25) (layer F.Cu) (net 9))
 (segment (start 139.7 94.361) (end 145.034 94.361) (width 0.25) (layer F.Cu) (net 9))
 (segment (start 138.049 96.012) (end 139.7 94.361) (width 0.25) (layer F.Cu) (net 9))
 (via (at 153.5 92.71) (size 0.6) (drill 0.4) (layers F.Cu B.Cu) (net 11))
 (segment (start 139.2235 90.2015) (end 139.192 90.17) (width 0.25) (layer F.Cu) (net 11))
 (via (at 139.192 90.17) (size 0.6) (drill 0.4) (layers F.Cu B.Cu) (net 11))
 (segment (start 148.082 90.17) (end 139.192 90.17) (width 0.25) (layer B.Cu) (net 11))
 (segment (start 150.495 92.583) (end 148.082 90.17) (width 0.25) (layer B.Cu) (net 11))
 (segment (start 153.373 92.583) (end 150.495 92.583) (width 0.25) (layer B.Cu) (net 11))
 (segment (start 153.373 92.583) (end 153.5 92.71) (width 0.25) (layer B.Cu) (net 11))
 (segment (start 151.765 85.09) (end 144.335 85.09) (width 0.25) (layer F.Cu) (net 11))
 (segment (start 144.335 85.09) (end 141.0015 88.4235) (width 0.25) (layer F.Cu) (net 11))
 (segment (start 141.0015 88.4235) (end 139.2235 90.2015) (width 0.25) (layer F.Cu) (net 11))
 (segment (start 139.2235 90.2015) (end 137.985 91.44) (width 0.25) (layer F.Cu) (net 11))
 (segment (start 151.3 76.2) (end 150.876 76.2) (width 0.25) (layer F.Cu) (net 23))
 (segment (start 150.876 76.2) (end 148.59 78.486) (width 0.25) (layer F.Cu) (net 23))
 (segment (start 148.59 78.486) (end 147.031 78.486) (width 0.25) (layer F.Cu) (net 23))
 (segment (start 147.031 78.486) (end 145.985 77.44) (width 0.25) (layer F.Cu) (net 23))
 (segment (start 143.985 77.44) (end 143.985 79.977) (width 0.25) (layer F.Cu) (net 24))
 (segment (start 153.5 89.365) (end 153.5 90.805) (width 0.25) (layer F.Cu) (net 24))
 (segment (start 153.162 89.027) (end 153.5 89.365) (width 0.25) (layer F.Cu) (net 24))
 (segment (start 151.13 89.027) (end 153.162 89.027) (width 0.25) (layer F.Cu) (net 24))
 (segment (start 150.241 88.138) (end 151.13 89.027) (width 0.25) (layer F.Cu) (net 24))
 (segment (start 147.828 85.725) (end 150.241 88.138) (width 0.25) (layer F.Cu) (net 24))
 (via (at 147.828 85.725) (size 0.6) (drill 0.4) (layers F.Cu B.Cu) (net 24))
 (segment (start 147.828 83.82) (end 147.828 85.725) (width 0.25) (layer B.Cu) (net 24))
 (segment (start 146.304 82.296) (end 147.828 83.82) (width 0.25) (layer B.Cu) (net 24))
 (via (at 146.304 82.296) (size 0.6) (drill 0.4) (layers F.Cu B.Cu) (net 24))
 (segment (start 143.985 79.977) (end 146.304 82.296) (width 0.25) (layer F.Cu) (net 24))
 (segment (start 141.985 77.44) (end 141.985 81.152) (width 0.25) (layer F.Cu) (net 12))
 (segment (start 144.653 83.82) (end 151.765 83.82) (width 0.25) (layer F.Cu) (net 12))
 (segment (start 141.985 81.152) (end 144.653 83.82) (width 0.25) (layer F.Cu) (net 12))
 (segment (start 158.115 85.09) (end 153.67 85.09) (width 0.25) (layer F.Cu) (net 17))
 (segment (start 133.985 78.613) (end 133.985 77.44) (width 0.25) (layer F.Cu) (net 17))
 (segment (start 134.62 79.248) (end 133.985 78.613) (width 0.25) (layer F.Cu) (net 17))
 (via (at 134.62 79.248) (size 0.6) (drill 0.4) (layers F.Cu B.Cu) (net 17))
 (segment (start 147.828 79.248) (end 134.62 79.248) (width 0.25) (layer B.Cu) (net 17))
 (segment (start 153.67 85.09) (end 147.828 79.248) (width 0.25) (layer B.Cu) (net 17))
 (via (at 153.67 85.09) (size 0.6) (drill 0.4) (layers F.Cu B.Cu) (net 17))
 (segment (start 135.985 77.44) (end 135.985 79.597) (width 0.25) (layer F.Cu) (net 18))
 (segment (start 153.67 86.36) (end 158.115 86.36) (width 0.25) (layer F.Cu) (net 18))
 (segment (start 153.543 86.487) (end 153.67 86.36) (width 0.25) (layer F.Cu) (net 18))
 (via (at 153.543 86.487) (size 0.6) (drill 0.4) (layers F.Cu B.Cu) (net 18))
 (segment (start 142.875 86.487) (end 153.543 86.487) (width 0.25) (layer B.Cu) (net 18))
 (segment (start 136.525 80.137) (end 142.875 86.487) (width 0.25) (layer B.Cu) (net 18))
 (via (at 136.525 80.137) (size 0.6) (drill 0.4) (layers F.Cu B.Cu) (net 18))
 (segment (start 135.985 79.597) (end 136.525 80.137) (width 0.25) (layer F.Cu) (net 18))
 (segment (start 132.17657 96.26368) (end 132.20932 96.26368) (width 0.25) (layer F.Cu) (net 10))
 (segment (start 132.20932 96.26368) (end 133.985 94.488) (width 0.25) (layer F.Cu) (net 10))
 (segment (start 133.985 94.488) (end 133.985 91.44) (width 0.25) (layer F.Cu) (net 10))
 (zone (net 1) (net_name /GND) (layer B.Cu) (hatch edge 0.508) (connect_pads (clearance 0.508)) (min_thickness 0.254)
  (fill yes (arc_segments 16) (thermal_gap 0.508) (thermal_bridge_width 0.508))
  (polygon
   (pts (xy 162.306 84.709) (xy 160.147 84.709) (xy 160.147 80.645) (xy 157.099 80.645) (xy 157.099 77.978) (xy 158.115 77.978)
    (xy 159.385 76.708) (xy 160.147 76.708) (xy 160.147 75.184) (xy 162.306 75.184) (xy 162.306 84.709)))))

